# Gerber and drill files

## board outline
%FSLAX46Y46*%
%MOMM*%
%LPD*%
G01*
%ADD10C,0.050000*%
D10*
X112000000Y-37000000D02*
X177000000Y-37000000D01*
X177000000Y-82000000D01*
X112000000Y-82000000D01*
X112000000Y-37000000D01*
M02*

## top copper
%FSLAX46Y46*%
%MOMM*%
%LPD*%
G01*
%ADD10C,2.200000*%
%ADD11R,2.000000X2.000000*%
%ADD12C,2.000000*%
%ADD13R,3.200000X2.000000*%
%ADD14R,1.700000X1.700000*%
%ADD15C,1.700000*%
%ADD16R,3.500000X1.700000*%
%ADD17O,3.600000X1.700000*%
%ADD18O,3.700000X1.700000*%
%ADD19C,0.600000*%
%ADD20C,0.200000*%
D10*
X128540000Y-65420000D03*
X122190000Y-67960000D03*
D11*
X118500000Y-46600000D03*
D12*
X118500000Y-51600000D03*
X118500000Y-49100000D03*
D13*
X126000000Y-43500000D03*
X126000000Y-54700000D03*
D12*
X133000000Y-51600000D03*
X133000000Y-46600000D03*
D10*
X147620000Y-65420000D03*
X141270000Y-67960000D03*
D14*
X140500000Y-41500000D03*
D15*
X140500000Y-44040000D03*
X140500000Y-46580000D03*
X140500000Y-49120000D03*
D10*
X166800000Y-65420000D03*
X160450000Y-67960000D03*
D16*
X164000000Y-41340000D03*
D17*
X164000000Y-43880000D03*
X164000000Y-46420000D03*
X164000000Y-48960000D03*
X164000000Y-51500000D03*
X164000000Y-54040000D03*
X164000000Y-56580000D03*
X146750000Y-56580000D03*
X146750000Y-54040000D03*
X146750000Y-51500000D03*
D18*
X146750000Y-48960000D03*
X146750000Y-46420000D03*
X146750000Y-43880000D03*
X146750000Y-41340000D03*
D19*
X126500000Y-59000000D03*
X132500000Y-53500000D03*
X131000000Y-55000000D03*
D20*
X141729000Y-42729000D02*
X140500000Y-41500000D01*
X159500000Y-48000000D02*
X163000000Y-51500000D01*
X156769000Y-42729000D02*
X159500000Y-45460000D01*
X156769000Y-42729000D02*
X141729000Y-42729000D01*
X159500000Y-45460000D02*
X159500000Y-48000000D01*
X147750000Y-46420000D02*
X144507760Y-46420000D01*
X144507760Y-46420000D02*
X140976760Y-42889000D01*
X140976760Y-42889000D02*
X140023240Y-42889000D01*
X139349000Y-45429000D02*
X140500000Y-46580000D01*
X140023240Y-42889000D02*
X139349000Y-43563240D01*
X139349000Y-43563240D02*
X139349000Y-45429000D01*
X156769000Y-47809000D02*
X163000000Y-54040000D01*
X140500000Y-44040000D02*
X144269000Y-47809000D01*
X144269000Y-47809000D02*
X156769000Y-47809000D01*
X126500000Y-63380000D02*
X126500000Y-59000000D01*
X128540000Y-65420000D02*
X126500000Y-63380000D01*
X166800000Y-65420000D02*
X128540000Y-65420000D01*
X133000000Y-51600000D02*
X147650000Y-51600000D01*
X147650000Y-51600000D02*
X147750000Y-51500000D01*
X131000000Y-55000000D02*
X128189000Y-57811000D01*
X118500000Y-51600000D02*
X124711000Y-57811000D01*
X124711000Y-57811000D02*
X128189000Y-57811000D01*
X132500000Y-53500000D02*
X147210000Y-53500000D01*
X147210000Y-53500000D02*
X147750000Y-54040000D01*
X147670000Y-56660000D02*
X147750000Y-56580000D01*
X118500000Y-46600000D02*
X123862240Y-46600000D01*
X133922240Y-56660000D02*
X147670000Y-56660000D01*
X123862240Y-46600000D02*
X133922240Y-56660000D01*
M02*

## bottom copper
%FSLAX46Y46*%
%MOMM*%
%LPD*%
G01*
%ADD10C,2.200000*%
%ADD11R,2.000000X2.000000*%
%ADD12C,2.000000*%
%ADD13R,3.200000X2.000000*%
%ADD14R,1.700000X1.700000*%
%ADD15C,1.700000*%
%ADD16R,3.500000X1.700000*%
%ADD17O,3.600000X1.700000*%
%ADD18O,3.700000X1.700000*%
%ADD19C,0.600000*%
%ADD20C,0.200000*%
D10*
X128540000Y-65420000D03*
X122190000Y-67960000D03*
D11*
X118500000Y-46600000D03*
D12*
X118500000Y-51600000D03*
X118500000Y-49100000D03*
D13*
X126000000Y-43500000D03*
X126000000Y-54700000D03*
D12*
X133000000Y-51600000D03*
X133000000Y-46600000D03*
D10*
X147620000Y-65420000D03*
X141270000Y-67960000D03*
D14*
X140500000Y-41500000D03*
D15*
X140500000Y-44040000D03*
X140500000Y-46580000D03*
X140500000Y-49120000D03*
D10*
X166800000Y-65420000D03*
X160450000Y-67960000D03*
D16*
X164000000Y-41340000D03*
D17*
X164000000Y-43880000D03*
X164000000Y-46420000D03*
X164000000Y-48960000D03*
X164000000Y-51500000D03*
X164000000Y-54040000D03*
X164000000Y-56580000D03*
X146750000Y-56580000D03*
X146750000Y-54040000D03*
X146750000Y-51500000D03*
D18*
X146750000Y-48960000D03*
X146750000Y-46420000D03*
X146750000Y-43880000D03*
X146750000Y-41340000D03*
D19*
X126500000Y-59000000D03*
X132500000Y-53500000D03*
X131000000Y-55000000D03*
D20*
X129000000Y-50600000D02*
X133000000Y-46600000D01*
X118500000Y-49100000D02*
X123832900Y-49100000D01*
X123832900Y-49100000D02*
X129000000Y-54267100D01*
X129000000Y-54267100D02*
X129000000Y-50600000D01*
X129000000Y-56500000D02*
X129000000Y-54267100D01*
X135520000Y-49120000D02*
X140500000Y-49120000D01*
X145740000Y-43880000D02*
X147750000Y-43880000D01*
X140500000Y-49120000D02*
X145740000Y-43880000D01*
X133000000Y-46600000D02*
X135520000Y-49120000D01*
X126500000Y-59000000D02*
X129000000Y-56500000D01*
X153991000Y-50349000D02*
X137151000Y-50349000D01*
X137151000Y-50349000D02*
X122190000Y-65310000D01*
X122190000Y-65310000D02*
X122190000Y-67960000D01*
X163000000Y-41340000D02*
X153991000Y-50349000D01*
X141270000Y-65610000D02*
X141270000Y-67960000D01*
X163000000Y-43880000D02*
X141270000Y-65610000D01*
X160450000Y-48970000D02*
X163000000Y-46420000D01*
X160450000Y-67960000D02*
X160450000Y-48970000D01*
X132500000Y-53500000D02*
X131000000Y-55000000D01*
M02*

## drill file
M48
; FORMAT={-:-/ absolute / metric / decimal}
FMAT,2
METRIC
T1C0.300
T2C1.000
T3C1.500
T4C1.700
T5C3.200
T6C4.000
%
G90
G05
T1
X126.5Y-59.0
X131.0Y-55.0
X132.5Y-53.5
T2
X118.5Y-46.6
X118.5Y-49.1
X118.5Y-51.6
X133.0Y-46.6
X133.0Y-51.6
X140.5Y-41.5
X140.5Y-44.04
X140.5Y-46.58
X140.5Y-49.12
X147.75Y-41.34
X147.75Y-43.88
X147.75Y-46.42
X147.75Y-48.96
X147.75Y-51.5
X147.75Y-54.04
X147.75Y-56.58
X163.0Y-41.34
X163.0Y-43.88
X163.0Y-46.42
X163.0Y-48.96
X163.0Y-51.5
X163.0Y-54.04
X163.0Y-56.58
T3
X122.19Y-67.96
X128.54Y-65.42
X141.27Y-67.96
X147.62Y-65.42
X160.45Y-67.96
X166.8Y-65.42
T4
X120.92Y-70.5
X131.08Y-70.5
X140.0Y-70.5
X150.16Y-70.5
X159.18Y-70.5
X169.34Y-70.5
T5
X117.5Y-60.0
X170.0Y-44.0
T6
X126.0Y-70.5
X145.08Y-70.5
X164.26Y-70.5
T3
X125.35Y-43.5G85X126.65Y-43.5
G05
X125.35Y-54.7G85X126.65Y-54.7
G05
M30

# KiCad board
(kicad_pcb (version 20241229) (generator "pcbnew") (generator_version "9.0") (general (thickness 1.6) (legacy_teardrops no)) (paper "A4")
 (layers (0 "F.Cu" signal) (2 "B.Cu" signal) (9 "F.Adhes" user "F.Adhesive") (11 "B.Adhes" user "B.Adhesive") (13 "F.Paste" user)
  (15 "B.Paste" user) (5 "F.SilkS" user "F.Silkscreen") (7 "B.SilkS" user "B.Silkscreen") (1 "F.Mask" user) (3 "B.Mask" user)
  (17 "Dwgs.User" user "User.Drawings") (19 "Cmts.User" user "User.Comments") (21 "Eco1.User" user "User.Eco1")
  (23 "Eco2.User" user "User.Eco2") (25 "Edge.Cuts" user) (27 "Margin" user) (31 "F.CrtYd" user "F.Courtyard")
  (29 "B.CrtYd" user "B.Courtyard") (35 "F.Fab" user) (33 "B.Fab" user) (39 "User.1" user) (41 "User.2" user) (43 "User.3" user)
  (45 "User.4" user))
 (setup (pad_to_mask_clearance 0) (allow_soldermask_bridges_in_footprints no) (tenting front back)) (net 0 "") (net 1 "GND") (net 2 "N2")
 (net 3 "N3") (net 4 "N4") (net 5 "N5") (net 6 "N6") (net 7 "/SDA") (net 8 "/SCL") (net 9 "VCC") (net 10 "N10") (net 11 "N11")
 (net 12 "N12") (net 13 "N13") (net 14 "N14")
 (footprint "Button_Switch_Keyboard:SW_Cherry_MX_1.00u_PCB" (layer "F.Cu") (at 128.54 65.42)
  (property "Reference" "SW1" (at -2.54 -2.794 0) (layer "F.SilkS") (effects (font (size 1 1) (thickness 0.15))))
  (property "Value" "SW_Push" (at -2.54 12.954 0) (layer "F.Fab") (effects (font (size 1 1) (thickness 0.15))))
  (pad "" np_thru_hole circle (at -7.62 5.08) (size 1.7 1.7) (drill 1.7) (layers "*.Cu" "*.Mask"))
  (pad "" np_thru_hole circle (at -2.54 5.08) (size 4 4) (drill 4) (layers "*.Cu" "*.Mask"))
  (pad "" np_thru_hole circle (at 2.54 5.08) (size 1.7 1.7) (drill 1.7) (layers "*.Cu" "*.Mask"))
  (pad "1" thru_hole circle (at 0 0) (size 2.2 2.2) (drill 1.5) (layers "*.Cu" "*.Mask") (remove_unused_layers no) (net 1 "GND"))
  (pad "2" thru_hole circle (at -6.35 2.54) (size 2.2 2.2) (drill 1.5) (layers "*.Cu" "*.Mask") (remove_unused_layers no) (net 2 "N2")))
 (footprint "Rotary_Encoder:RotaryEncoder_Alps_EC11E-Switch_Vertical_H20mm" (layer "F.Cu") (at 118.5 46.6)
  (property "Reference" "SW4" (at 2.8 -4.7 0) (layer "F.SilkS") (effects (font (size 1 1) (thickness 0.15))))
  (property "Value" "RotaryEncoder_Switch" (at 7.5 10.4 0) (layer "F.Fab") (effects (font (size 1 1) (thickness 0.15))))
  (pad "A" thru_hole rect (at 0 0) (size 2 2) (drill 1) (layers "*.Cu" "*.Mask") (remove_unused_layers no) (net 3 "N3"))
  (pad "B" thru_hole circle (at 0 5) (size 2 2) (drill 1) (layers "*.Cu" "*.Mask") (remove_unused_layers no) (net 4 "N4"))
  (pad "C" thru_hole circle (at 0 2.5) (size 2 2) (drill 1) (layers "*.Cu" "*.Mask") (remove_unused_layers no) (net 1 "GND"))
  (pad "MP" thru_hole rect (at 7.5 -3.1) (size 3.2 2) (drill oval 2.8 1.5) (layers "*.Cu" "*.Mask") (remove_unused_layers no))
  (pad "MP" thru_hole rect (at 7.5 8.1) (size 3.2 2) (drill oval 2.8 1.5) (layers "*.Cu" "*.Mask") (remove_unused_layers no))
  (pad "S1" thru_hole circle (at 14.5 5) (size 2 2) (drill 1) (layers "*.Cu" "*.Mask") (remove_unused_layers no) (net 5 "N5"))
  (pad "S2" thru_hole circle (at 14.5 0) (size 2 2) (drill 1) (layers "*.Cu" "*.Mask") (remove_unused_layers no) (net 1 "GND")))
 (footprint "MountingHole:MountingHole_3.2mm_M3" (layer "F.Cu") (at 117.5 60)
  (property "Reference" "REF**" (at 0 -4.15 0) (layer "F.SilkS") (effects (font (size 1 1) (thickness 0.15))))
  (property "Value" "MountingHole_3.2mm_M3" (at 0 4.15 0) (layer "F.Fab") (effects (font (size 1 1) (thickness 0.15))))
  (pad "" np_thru_hole circle (at 0 0) (size 3.2 3.2) (drill 3.2) (layers "*.Cu" "*.Mask")))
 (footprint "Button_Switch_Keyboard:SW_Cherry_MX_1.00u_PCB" (layer "F.Cu") (at 147.62 65.42)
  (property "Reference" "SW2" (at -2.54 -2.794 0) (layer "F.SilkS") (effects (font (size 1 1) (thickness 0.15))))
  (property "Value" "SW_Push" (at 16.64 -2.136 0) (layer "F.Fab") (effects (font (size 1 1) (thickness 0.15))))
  (pad "" np_thru_hole circle (at -7.62 5.08) (size 1.7 1.7) (drill 1.7) (layers "*.Cu" "*.Mask"))
  (pad "" np_thru_hole circle (at -2.54 5.08) (size 4 4) (drill 4) (layers "*.Cu" "*.Mask"))
  (pad "" np_thru_hole circle (at 2.54 5.08) (size 1.7 1.7) (drill 1.7) (layers "*.Cu" "*.Mask"))
  (pad "1" thru_hole circle (at 0 0) (size 2.2 2.2) (drill 1.5) (layers "*.Cu" "*.Mask") (remove_unused_layers no) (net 1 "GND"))
  (pad "2" thru_hole circle (at -6.35 2.54) (size 2.2 2.2) (drill 1.5) (layers "*.Cu" "*.Mask") (remove_unused_layers no) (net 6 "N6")))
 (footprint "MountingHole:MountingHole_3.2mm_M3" (layer "F.Cu") (at 170 44)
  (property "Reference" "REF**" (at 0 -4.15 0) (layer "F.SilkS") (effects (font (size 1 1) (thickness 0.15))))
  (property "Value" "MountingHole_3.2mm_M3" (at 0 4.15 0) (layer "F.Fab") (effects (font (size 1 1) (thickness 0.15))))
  (pad "" np_thru_hole circle (at 0 0) (size 3.2 3.2) (drill 3.2) (layers "*.Cu" "*.Mask")))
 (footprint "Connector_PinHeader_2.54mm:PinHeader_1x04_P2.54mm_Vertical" (layer "F.Cu") (at 140.5 41.5)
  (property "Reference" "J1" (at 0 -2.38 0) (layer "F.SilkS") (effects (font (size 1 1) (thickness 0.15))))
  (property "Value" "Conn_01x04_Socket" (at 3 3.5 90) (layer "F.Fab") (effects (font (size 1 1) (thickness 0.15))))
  (pad "1" thru_hole rect (at 0 0) (size 1.7 1.7) (drill 1) (layers "*.Cu" "*.Mask") (remove_unused_layers no) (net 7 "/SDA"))
  (pad "2" thru_hole circle (at 0 2.54) (size 1.7 1.7) (drill 1) (layers "*.Cu" "*.Mask") (remove_unused_layers no) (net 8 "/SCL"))
  (pad "3" thru_hole circle (at 0 5.08) (size 1.7 1.7) (drill 1) (layers "*.Cu" "*.Mask") (remove_unused_layers no) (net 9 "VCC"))
  (pad "4" thru_hole circle (at 0 7.62) (size 1.7 1.7) (drill 1) (layers "*.Cu" "*.Mask") (remove_unused_layers no) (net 1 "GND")))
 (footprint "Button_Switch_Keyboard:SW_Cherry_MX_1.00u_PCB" (layer "F.Cu") (at 166.8 65.42)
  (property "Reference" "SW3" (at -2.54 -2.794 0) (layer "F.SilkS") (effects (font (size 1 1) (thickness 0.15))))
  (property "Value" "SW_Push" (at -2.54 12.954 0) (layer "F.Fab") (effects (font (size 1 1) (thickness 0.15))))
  (pad "" np_thru_hole circle (at -7.62 5.08) (size 1.7 1.7) (drill 1.7) (layers "*.Cu" "*.Mask"))
  (pad "" np_thru_hole circle (at -2.54 5.08) (size 4 4) (drill 4) (layers "*.Cu" "*.Mask"))
  (pad "" np_thru_hole circle (at 2.54 5.08) (size 1.7 1.7) (drill 1.7) (layers "*.Cu" "*.Mask"))
  (pad "1" thru_hole circle (at 0 0) (size 2.2 2.2) (drill 1.5) (layers "*.Cu" "*.Mask") (remove_unused_layers no) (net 1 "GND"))
  (pad "2" thru_hole circle (at -6.35 2.54) (size 2.2 2.2) (drill 1.5) (layers "*.Cu" "*.Mask") (remove_unused_layers no) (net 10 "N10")))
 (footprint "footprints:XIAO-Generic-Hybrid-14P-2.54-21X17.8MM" (layer "B.Cu") (at 155.375 48.96 180)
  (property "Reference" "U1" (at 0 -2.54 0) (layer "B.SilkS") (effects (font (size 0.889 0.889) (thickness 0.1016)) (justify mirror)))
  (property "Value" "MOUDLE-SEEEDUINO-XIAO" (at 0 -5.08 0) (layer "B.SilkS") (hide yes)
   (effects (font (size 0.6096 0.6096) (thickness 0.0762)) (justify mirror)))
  (pad "1" thru_hole rect (at -7.625 7.62 180) (size 3.5 1.7) (drill 1 (offset -1 0)) (layers "*.Cu" "*.Mask") (remove_unused_layers no)
   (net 2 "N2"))
  (pad "2" thru_hole oval (at -7.625 5.08 180) (size 3.6 1.7) (drill 1 (offset -1 0)) (layers "*.Cu" "*.Mask") (remove_unused_layers no)
   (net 6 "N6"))
  (pad "3" thru_hole oval (at -7.625 2.54 180) (size 3.6 1.7) (drill 1 (offset -1 0)) (layers "*.Cu" "*.Mask") (remove_unused_layers no)
   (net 10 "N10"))
  (pad "4" thru_hole oval (at -7.625 0 180) (size 3.6 1.7) (drill 1 (offset -1 0)) (layers "*.Cu" "*.Mask") (remove_unused_layers no)
   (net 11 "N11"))
  (pad "5" thru_hole oval (at -7.625 -2.54 180) (size 3.6 1.7) (drill 1 (offset -1 0)) (layers "*.Cu" "*.Mask") (remove_unused_layers no)
   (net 7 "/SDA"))
  (pad "6" thru_hole oval (at -7.625 -5.08) (size 3.6 1.7) (drill 1 (offset 1 0)) (layers "*.Cu" "*.Mask") (remove_unused_layers no)
   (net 8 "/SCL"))
  (pad "7" thru_hole oval (at -7.625 -7.62 180) (size 3.6 1.7) (drill 1 (offset -1 0)) (layers "*.Cu" "*.Mask") (remove_unused_layers no)
   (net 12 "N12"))
  (pad "8" thru_hole oval (at 7.625 -7.62 180) (size 3.6 1.7) (drill 1 (offset 1 0)) (layers "*.Cu" "*.Mask") (remove_unused_layers no)
   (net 3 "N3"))
  (pad "9" thru_hole oval (at 7.625 -5.08 180) (size 3.6 1.7) (drill 1 (offset 1 0)) (layers "*.Cu" "*.Mask") (remove_unused_layers no)
   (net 4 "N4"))
  (pad "10" thru_hole oval (at 7.625 -2.54 180) (size 3.6 1.7) (drill 1 (offset 1 0)) (layers "*.Cu" "*.Mask") (remove_unused_layers no)
   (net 5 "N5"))
  (pad "11" thru_hole oval (at 7.625 0 180) (size 3.7 1.7) (drill 1 (offset 1 0)) (layers "*.Cu" "*.Mask") (remove_unused_layers no)
   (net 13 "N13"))
  (pad "12" thru_hole oval (at 7.625 2.54 180) (size 3.7 1.7) (drill 1 (offset 1 0)) (layers "*.Cu" "*.Mask") (remove_unused_layers no)
   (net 9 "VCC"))
  (pad "13" thru_hole oval (at 7.625 5.08 180) (size 3.7 1.7) (drill 1 (offset 1 0)) (layers "*.Cu" "*.Mask") (remove_unused_layers no)
   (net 1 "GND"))
  (pad "14" thru_hole oval (at 7.625 7.62 180) (size 3.7 1.7) (drill 1 (offset 1 0)) (layers "*.Cu" "*.Mask") (remove_unused_layers no)
   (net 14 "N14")))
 (gr_rect (start 112 37) (end 177 82) (stroke (width 0.05) (type default)) (fill no) (layer "Edge.Cuts"))
 (segment (start 141.729 42.729) (end 140.5 41.5) (width 0.2) (layer "F.Cu") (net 7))
 (segment (start 159.5 48) (end 163 51.5) (width 0.2) (layer "F.Cu") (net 7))
 (segment (start 156.769 42.729) (end 159.5 45.46) (width 0.2) (layer "F.Cu") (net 7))
 (segment (start 156.769 42.729) (end 141.729 42.729) (width 0.2) (layer "F.Cu") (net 7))
 (segment (start 159.5 45.46) (end 159.5 48) (width 0.2) (layer "F.Cu") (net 7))
 (segment (start 147.75 46.42) (end 144.50776 46.42) (width 0.2) (layer "F.Cu") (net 9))
 (segment (start 144.50776 46.42) (end 140.97676 42.889) (width 0.2) (layer "F.Cu") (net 9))
 (segment (start 140.97676 42.889) (end 140.02324 42.889) (width 0.2) (layer "F.Cu") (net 9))
 (segment (start 139.349 45.429) (end 140.5 46.58) (width 0.2) (layer "F.Cu") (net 9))
 (segment (start 140.02324 42.889) (end 139.349 43.56324) (width 0.2) (layer "F.Cu") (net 9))
 (segment (start 139.349 43.56324) (end 139.349 45.429) (width 0.2) (layer "F.Cu") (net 9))
 (segment (start 156.769 47.809) (end 163 54.04) (width 0.2) (layer "F.Cu") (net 8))
 (segment (start 140.5 44.04) (end 144.269 47.809) (width 0.2) (layer "F.Cu") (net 8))
 (segment (start 144.269 47.809) (end 156.769 47.809) (width 0.2) (layer "F.Cu") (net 8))
 (segment (start 126.5 63.38) (end 126.5 59) (width 0.2) (layer "F.Cu") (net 1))
 (segment (start 128.54 65.42) (end 126.5 63.38) (width 0.2) (layer "F.Cu") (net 1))
 (segment (start 166.8 65.42) (end 128.54 65.42) (width 0.2) (layer "F.Cu") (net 1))
 (via (at 126.5 59) (size 0.6) (drill 0.3) (layers "F.Cu" "B.Cu") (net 1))
 (segment (start 129 50.6) (end 133 46.6) (width 0.2) (layer "B.Cu") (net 1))
 (segment (start 118.5 49.1) (end 123.8329 49.1) (width 0.2) (layer "B.Cu") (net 1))
 (segment (start 123.8329 49.1) (end 129 54.2671) (width 0.2) (layer "B.Cu") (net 1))
 (segment (start 129 54.2671) (end 129 50.6) (width 0.2) (layer "B.Cu") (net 1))
 (segment (start 129 56.5) (end 129 54.2671) (width 0.2) (layer "B.Cu") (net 1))
 (segment (start 135.52 49.12) (end 140.5 49.12) (width 0.2) (layer "B.Cu") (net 1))
 (segment (start 145.74 43.88) (end 147.75 43.88) (width 0.2) (layer "B.Cu") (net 1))
 (segment (start 140.5 49.12) (end 145.74 43.88) (width 0.2) (layer "B.Cu") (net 1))
 (segment (start 133 46.6) (end 135.52 49.12) (width 0.2) (layer "B.Cu") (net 1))
 (segment (start 126.5 59) (end 129 56.5) (width 0.2) (layer "B.Cu") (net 1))
 (segment (start 153.991 50.349) (end 137.151 50.349) (width 0.2) (layer "B.Cu") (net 2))
 (segment (start 137.151 50.349) (end 122.19 65.31) (width 0.2) (layer "B.Cu") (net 2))
 (segment (start 122.19 65.31) (end 122.19 67.96) (width 0.2) (layer "B.Cu") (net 2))
 (segment (start 163 41.34) (end 153.991 50.349) (width 0.2) (layer "B.Cu") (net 2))
 (segment (start 141.27 65.61) (end 141.27 67.96) (width 0.2) (layer "B.Cu") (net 6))
 (segment (start 163 43.88) (end 141.27 65.61) (width 0.2) (layer "B.Cu") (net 6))
 (segment (start 160.45 48.97) (end 163 46.42) (width 0.2) (layer "B.Cu") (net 10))
 (segment (start 160.45 67.96) (end 160.45 48.97) (width 0.2) (layer "B.Cu") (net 10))
 (segment (start 133 51.6) (end 147.65 51.6) (width 0.2) (layer "F.Cu") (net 5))
 (segment (start 147.65 51.6) (end 147.75 51.5) (width 0.2) (layer "F.Cu") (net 5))
 (segment (start 131 55) (end 128.189 57.811) (width 0.2) (layer "F.Cu") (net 4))
 (segment (start 118.5 51.6) (end 124.711 57.811) (width 0.2) (layer "F.Cu") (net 4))
 (segment (start 124.711 57.811) (end 128.189 57.811) (width 0.2) (layer "F.Cu") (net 4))
 (segment (start 132.5 53.5) (end 147.21 53.5) (width 0.2) (layer "F.Cu") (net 4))
 (segment (start 147.21 53.5) (end 147.75 54.04) (width 0.2) (layer "F.Cu") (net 4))
 (via (at 132.5 53.5) (size 0.6) (drill 0.3) (layers "F.Cu" "B.Cu") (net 4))
 (via (at 131 55) (size 0.6) (drill 0.3) (layers "F.Cu" "B.Cu") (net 4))
 (segment (start 132.5 53.5) (end 131 55) (width 0.2) (layer "B.Cu") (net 4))
 (segment (start 147.67 56.66) (end 147.75 56.58) (width 0.2) (layer "F.Cu") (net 3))
 (segment (start 118.5 46.6) (end 123.86224 46.6) (width 0.2) (layer "F.Cu") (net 3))
 (segment (start 133.92224 56.66) (end 147.67 56.66) (width 0.2) (layer "F.Cu") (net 3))
 (segment (start 123.86224 46.6) (end 133.92224 56.66) (width 0.2) (layer "F.Cu") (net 3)))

